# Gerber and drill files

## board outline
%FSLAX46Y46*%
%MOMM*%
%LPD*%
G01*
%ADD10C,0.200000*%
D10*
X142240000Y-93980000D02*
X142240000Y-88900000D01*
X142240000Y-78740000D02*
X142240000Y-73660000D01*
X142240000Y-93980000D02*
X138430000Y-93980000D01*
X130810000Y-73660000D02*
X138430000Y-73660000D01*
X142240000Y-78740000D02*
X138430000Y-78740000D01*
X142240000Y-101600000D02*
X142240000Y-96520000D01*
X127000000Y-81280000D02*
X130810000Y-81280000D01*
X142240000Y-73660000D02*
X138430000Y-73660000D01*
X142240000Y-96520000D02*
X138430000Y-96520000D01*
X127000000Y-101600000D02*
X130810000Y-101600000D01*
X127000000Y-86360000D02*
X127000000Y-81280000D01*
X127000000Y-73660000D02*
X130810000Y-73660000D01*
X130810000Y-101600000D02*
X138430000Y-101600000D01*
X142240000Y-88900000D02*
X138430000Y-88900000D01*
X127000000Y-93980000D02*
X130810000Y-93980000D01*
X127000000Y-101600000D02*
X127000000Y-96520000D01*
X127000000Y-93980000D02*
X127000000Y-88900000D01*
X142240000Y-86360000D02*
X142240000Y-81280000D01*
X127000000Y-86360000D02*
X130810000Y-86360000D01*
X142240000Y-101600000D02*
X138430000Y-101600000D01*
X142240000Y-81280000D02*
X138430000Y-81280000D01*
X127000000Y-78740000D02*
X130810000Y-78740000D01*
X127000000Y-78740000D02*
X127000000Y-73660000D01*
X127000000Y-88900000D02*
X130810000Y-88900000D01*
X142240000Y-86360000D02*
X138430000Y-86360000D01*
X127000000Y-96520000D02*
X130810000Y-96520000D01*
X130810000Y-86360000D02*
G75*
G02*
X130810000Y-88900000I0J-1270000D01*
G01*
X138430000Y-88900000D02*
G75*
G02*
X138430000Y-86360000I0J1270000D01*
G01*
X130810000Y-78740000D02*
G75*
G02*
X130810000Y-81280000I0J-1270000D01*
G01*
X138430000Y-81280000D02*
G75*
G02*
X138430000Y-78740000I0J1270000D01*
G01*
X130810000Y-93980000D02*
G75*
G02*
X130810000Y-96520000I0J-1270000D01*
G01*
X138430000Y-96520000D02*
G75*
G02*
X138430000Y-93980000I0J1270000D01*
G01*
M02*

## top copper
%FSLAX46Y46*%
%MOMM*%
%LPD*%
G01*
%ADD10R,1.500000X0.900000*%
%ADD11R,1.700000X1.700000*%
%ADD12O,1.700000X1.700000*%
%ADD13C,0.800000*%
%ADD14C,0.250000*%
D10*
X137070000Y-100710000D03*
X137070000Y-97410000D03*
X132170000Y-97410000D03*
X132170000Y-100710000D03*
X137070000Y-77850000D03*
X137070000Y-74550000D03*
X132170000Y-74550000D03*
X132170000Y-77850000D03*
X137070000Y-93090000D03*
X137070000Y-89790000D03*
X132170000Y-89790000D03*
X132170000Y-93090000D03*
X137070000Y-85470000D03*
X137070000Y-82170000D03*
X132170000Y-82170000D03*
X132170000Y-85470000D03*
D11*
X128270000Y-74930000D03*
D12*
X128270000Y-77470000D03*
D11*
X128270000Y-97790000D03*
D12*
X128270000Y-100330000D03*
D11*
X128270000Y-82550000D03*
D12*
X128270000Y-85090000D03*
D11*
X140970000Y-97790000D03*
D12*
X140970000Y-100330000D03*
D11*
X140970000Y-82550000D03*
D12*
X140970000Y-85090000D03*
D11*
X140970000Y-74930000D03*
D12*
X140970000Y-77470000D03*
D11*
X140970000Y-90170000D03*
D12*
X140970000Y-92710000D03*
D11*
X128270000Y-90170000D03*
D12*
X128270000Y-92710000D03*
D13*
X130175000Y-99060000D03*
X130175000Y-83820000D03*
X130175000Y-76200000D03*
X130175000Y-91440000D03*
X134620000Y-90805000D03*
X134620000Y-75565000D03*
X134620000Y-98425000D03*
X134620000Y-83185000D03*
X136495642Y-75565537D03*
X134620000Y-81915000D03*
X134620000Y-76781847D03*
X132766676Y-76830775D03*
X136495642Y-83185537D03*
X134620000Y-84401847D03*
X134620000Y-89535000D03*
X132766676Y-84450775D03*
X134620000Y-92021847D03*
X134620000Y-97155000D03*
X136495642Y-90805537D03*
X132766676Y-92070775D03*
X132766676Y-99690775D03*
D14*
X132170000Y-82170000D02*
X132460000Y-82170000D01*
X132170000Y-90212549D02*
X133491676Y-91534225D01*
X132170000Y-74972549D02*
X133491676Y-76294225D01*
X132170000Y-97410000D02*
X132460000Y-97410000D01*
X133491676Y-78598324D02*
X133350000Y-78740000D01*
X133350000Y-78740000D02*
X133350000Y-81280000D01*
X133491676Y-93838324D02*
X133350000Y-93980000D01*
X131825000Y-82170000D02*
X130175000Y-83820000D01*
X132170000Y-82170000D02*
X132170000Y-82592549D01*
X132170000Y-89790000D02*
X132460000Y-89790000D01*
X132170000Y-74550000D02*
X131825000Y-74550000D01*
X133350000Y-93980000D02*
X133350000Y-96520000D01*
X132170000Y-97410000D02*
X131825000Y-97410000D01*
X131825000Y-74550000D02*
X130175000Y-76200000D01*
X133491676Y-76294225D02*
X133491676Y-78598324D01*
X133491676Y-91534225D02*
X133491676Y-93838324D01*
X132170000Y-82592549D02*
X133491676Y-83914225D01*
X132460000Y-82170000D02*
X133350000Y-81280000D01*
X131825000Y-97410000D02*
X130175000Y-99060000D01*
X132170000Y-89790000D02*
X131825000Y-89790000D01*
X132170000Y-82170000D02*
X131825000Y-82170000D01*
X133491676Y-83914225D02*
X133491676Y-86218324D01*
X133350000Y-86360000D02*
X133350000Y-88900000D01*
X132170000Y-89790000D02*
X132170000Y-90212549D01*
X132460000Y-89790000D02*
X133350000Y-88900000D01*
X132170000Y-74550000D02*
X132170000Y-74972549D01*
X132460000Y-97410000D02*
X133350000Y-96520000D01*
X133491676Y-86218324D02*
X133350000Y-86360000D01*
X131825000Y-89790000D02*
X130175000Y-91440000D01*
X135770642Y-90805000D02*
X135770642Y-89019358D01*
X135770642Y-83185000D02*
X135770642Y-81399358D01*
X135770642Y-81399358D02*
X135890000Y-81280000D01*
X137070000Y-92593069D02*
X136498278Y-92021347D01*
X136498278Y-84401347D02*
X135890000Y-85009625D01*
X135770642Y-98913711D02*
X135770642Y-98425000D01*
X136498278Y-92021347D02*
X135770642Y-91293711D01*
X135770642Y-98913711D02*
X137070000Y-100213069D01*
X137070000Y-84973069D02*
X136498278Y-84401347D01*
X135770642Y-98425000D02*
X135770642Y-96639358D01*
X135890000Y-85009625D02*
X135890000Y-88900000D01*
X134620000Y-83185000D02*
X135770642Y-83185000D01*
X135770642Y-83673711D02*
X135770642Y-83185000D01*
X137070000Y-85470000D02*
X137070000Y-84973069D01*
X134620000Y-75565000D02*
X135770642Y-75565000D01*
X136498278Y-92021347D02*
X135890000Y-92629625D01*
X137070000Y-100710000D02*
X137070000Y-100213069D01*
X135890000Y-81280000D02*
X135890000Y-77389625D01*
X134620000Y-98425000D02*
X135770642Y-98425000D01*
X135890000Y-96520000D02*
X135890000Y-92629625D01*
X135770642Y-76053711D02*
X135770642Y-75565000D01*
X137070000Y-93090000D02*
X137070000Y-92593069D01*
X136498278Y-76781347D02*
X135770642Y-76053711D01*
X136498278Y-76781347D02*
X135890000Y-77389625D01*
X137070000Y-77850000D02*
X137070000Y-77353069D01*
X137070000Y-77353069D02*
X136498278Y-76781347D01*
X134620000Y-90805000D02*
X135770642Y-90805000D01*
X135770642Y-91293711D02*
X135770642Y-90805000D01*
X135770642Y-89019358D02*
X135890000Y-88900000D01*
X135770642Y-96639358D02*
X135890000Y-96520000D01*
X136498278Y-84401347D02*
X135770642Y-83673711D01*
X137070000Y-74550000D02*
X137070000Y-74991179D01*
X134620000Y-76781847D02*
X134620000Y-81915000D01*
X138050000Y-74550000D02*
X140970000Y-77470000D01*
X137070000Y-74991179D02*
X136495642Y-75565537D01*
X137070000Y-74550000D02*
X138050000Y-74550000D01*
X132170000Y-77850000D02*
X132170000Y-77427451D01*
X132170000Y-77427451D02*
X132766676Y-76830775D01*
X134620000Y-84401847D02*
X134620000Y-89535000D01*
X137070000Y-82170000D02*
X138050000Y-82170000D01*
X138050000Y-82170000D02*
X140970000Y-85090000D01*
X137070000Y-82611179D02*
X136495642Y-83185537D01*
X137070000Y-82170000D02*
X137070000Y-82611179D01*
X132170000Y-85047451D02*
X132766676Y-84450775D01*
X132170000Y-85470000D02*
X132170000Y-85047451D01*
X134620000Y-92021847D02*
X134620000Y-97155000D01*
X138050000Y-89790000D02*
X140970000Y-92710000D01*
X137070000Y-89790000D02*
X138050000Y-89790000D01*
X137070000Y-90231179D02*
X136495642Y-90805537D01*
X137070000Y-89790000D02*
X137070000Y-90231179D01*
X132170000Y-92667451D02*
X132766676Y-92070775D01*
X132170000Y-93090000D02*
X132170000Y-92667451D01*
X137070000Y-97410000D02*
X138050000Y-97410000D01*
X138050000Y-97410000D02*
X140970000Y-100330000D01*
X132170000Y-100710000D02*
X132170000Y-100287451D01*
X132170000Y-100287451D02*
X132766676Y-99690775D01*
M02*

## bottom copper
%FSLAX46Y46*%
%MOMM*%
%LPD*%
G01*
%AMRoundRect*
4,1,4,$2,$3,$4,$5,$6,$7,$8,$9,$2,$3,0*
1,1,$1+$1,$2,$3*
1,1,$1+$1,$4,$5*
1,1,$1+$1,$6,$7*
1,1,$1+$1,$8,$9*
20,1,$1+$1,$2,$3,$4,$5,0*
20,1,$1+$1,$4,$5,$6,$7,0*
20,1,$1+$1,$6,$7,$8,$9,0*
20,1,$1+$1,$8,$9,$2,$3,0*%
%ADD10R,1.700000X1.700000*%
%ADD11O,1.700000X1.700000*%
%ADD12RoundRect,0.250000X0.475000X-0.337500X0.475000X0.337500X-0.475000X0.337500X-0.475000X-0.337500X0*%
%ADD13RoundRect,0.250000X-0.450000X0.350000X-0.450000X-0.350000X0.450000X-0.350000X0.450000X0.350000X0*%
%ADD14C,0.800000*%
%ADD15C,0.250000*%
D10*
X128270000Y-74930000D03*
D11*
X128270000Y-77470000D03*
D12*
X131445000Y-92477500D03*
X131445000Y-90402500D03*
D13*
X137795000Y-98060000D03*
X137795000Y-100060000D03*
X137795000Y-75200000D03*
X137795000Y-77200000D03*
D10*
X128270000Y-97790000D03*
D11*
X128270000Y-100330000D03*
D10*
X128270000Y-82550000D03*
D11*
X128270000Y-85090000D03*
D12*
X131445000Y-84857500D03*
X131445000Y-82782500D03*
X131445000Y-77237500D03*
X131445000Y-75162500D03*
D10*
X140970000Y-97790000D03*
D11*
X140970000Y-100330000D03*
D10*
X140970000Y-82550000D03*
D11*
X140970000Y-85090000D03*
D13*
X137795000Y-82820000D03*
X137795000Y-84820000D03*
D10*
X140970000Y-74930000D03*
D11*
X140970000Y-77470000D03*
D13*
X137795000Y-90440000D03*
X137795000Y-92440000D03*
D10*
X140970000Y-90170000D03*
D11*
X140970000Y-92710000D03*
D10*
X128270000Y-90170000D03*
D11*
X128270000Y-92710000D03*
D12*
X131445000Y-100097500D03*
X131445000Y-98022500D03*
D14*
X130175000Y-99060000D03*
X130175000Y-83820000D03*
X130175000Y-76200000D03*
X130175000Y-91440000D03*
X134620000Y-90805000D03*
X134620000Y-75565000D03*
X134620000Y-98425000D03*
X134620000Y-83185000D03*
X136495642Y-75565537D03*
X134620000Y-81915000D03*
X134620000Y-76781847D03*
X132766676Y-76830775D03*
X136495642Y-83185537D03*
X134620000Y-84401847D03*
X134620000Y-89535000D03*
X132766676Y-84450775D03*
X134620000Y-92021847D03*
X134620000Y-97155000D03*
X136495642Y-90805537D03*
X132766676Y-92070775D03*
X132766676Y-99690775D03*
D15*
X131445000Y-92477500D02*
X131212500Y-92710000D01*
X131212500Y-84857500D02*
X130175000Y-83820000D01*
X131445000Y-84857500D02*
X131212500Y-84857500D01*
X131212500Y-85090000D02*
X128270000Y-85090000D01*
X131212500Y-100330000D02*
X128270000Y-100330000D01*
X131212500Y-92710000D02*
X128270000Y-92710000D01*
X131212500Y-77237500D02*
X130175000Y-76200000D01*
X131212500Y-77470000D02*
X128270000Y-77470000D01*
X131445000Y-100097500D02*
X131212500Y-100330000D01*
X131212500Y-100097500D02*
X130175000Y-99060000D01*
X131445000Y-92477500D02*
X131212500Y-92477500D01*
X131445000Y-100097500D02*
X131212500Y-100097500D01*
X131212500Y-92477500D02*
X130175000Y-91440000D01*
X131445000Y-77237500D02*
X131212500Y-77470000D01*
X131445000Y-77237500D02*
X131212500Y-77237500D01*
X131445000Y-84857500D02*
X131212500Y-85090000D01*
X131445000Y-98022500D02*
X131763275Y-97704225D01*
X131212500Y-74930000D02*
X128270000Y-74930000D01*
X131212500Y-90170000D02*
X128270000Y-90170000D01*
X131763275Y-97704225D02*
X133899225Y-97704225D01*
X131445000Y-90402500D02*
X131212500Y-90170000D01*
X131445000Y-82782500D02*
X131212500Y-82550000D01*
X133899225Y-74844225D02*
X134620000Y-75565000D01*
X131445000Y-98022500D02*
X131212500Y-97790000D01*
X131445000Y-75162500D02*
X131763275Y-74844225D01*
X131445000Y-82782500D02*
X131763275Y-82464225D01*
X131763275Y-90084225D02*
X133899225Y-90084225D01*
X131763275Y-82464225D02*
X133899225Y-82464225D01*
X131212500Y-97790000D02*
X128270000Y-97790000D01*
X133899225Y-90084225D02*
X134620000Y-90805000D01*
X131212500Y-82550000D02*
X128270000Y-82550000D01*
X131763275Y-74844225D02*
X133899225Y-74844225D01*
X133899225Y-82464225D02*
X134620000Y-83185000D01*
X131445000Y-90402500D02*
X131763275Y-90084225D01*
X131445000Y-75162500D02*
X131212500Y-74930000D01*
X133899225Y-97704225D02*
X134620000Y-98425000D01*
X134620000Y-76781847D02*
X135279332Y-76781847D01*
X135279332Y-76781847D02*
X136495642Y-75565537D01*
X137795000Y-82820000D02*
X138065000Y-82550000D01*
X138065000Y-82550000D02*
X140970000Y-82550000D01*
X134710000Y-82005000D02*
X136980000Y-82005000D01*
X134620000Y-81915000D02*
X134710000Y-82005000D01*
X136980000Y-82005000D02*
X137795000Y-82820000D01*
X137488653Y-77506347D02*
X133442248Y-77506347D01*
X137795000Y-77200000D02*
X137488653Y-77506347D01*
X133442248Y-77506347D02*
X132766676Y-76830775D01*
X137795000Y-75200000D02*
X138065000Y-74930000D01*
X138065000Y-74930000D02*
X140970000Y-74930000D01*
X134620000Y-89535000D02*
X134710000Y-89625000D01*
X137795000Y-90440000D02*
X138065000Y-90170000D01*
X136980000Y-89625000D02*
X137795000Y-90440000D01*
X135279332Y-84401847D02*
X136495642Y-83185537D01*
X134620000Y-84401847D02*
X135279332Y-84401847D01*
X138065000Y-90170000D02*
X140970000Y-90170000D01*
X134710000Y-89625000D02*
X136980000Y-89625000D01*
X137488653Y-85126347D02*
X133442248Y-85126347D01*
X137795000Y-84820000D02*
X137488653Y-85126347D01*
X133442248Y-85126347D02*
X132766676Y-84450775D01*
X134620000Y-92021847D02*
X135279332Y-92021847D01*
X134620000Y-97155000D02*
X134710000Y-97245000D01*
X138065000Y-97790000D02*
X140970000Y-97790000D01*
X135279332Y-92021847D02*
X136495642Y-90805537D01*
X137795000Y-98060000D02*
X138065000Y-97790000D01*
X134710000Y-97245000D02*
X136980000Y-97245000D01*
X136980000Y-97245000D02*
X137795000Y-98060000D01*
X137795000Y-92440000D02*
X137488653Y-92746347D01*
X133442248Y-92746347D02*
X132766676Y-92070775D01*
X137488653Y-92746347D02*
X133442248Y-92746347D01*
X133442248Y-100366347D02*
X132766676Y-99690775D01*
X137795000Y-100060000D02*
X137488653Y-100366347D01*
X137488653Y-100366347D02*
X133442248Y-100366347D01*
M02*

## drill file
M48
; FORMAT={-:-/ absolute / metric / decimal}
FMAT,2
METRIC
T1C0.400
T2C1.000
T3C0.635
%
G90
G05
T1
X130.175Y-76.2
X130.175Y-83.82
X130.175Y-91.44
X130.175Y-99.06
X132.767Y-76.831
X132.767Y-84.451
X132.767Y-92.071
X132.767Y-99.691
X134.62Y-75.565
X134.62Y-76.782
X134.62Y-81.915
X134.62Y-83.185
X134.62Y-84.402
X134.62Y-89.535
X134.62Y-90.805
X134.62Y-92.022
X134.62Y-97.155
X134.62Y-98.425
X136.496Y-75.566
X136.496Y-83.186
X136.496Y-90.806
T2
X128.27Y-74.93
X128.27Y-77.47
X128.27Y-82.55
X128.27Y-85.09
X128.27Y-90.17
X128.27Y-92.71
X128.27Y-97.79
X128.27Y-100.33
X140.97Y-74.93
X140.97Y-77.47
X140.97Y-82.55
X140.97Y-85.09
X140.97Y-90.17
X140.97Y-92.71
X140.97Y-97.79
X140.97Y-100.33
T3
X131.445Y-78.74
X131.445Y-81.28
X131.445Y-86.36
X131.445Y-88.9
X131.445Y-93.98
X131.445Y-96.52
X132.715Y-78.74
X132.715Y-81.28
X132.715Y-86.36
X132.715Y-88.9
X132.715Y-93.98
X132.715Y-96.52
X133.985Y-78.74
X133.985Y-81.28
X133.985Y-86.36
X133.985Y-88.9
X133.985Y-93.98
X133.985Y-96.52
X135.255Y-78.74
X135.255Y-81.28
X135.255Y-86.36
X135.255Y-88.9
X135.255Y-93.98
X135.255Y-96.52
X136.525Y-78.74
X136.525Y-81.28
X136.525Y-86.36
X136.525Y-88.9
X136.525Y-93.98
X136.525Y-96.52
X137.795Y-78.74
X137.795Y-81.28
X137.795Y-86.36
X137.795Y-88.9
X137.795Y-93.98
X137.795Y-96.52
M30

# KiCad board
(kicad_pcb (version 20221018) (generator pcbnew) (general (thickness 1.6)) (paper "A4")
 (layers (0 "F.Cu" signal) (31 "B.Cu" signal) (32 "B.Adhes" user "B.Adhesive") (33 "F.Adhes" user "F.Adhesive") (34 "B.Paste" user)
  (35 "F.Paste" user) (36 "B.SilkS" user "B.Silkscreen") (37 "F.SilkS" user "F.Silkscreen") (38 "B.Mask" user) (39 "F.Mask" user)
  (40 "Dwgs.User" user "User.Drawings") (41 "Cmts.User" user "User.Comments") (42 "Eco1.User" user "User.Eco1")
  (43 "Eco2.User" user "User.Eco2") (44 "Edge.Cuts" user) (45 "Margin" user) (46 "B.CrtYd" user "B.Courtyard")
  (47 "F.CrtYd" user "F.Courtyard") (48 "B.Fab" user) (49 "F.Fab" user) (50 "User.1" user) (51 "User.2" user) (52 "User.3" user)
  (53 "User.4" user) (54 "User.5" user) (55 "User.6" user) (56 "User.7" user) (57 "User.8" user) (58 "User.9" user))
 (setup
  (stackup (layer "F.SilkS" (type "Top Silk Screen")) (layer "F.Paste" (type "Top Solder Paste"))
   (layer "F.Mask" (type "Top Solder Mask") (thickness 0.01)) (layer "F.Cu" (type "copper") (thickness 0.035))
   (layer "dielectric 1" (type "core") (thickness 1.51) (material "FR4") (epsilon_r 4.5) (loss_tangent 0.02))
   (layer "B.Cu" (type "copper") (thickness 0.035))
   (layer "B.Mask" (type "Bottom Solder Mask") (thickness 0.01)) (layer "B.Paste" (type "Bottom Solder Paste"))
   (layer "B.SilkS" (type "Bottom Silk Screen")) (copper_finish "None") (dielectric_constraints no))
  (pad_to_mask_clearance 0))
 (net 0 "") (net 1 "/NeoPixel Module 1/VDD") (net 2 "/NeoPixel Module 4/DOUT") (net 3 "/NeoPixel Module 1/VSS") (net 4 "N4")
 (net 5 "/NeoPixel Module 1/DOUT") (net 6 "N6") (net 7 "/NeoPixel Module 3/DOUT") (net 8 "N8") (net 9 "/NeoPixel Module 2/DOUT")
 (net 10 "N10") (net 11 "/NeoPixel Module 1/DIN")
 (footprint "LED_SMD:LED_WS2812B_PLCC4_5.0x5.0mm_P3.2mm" (layer "F.Cu") (at 134.62 99.06 180)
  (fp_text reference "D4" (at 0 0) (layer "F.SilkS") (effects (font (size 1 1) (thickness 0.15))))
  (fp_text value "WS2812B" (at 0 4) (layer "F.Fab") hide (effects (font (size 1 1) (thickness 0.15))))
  (pad "1" smd rect (at -2.45 -1.65 180) (size 1.5 0.9) (layers "F.Cu" "F.Paste" "F.Mask") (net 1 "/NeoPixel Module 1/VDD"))
  (pad "2" smd rect (at -2.45 1.65 180) (size 1.5 0.9) (layers "F.Cu" "F.Paste" "F.Mask") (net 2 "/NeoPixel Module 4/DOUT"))
  (pad "3" smd rect (at 2.45 1.65 180) (size 1.5 0.9) (layers "F.Cu" "F.Paste" "F.Mask") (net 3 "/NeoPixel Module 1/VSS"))
  (pad "4" smd rect (at 2.45 -1.65 180) (size 1.5 0.9) (layers "F.Cu" "F.Paste" "F.Mask") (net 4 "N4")))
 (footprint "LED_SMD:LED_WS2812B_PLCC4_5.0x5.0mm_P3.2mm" (layer "F.Cu") (at 134.62 76.2 180)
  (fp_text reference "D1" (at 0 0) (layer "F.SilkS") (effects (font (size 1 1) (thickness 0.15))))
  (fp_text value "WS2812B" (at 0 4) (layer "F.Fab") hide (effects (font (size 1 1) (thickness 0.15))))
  (pad "1" smd rect (at -2.45 -1.65 180) (size 1.5 0.9) (layers "F.Cu" "F.Paste" "F.Mask") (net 1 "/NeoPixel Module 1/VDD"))
  (pad "2" smd rect (at -2.45 1.65 180) (size 1.5 0.9) (layers "F.Cu" "F.Paste" "F.Mask") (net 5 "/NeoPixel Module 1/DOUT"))
  (pad "3" smd rect (at 2.45 1.65 180) (size 1.5 0.9) (layers "F.Cu" "F.Paste" "F.Mask") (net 3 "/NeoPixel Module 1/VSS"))
  (pad "4" smd rect (at 2.45 -1.65 180) (size 1.5 0.9) (layers "F.Cu" "F.Paste" "F.Mask") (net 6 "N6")))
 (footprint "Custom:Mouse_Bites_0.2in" (layer "F.Cu") (at 134.62 87.63)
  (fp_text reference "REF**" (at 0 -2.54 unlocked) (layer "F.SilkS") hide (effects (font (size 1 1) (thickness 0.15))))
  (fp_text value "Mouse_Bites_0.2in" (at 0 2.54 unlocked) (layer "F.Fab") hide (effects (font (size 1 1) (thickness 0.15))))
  (fp_arc (start -3.81 -1.27) (mid -2.54 0) (end -3.81 1.27) (stroke (width 0.2) (type default)) (layer "Edge.Cuts"))
  (fp_arc (start 3.81 1.27) (mid 2.54 0) (end 3.81 -1.27) (stroke (width 0.2) (type default)) (layer "Edge.Cuts"))
  (pad "" np_thru_hole circle (at -3.175 -1.27) (size 0.635 0.635) (drill 0.635) (layers "*.Mask") (thermal_bridge_angle 90))
  (pad "" np_thru_hole circle (at -3.175 1.27) (size 0.635 0.635) (drill 0.635) (layers "*.Mask") (thermal_bridge_angle 90))
  (pad "" np_thru_hole circle (at -1.905 -1.27) (size 0.635 0.635) (drill 0.635) (layers "*.Mask") (thermal_bridge_angle 90))
  (pad "" np_thru_hole circle (at -1.905 1.27) (size 0.635 0.635) (drill 0.635) (layers "*.Mask") (thermal_bridge_angle 90))
  (pad "" np_thru_hole circle (at -0.635 -1.27) (size 0.635 0.635) (drill 0.635) (layers "*.Mask") (thermal_bridge_angle 90))
  (pad "" np_thru_hole circle (at -0.635 1.27) (size 0.635 0.635) (drill 0.635) (layers "*.Mask") (thermal_bridge_angle 90))
  (pad "" np_thru_hole circle (at 0.635 -1.27) (size 0.635 0.635) (drill 0.635) (layers "*.Mask") (thermal_bridge_angle 90))
  (pad "" np_thru_hole circle (at 0.635 1.27) (size 0.635 0.635) (drill 0.635) (layers "*.Mask") (thermal_bridge_angle 90))
  (pad "" np_thru_hole circle (at 1.905 -1.27) (size 0.635 0.635) (drill 0.635) (layers "*.Mask") (thermal_bridge_angle 90))
  (pad "" np_thru_hole circle (at 1.905 1.27) (size 0.635 0.635) (drill 0.635) (layers "*.Mask") (thermal_bridge_angle 90))
  (pad "" np_thru_hole circle (at 3.175 -1.27) (size 0.635 0.635) (drill 0.635) (layers "*.Mask") (thermal_bridge_angle 90))
  (pad "" np_thru_hole circle (at 3.175 1.27) (size 0.635 0.635) (drill 0.635) (layers "*.Mask") (thermal_bridge_angle 90)))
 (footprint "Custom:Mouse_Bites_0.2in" (layer "F.Cu") (at 134.62 80.01)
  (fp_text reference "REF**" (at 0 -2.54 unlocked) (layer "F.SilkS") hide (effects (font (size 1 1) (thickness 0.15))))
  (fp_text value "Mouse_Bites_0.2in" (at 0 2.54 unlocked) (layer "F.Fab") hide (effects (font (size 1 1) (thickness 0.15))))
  (fp_arc (start -3.81 -1.27) (mid -2.54 0) (end -3.81 1.27) (stroke (width 0.2) (type default)) (layer "Edge.Cuts"))
  (fp_arc (start 3.81 1.27) (mid 2.54 0) (end 3.81 -1.27) (stroke (width 0.2) (type default)) (layer "Edge.Cuts"))
  (pad "" np_thru_hole circle (at -3.175 -1.27) (size 0.635 0.635) (drill 0.635) (layers "*.Mask") (thermal_bridge_angle 90))
  (pad "" np_thru_hole circle (at -3.175 1.27) (size 0.635 0.635) (drill 0.635) (layers "*.Mask") (thermal_bridge_angle 90))
  (pad "" np_thru_hole circle (at -1.905 -1.27) (size 0.635 0.635) (drill 0.635) (layers "*.Mask") (thermal_bridge_angle 90))
  (pad "" np_thru_hole circle (at -1.905 1.27) (size 0.635 0.635) (drill 0.635) (layers "*.Mask") (thermal_bridge_angle 90))
  (pad "" np_thru_hole circle (at -0.635 -1.27) (size 0.635 0.635) (drill 0.635) (layers "*.Mask") (thermal_bridge_angle 90))
  (pad "" np_thru_hole circle (at -0.635 1.27) (size 0.635 0.635) (drill 0.635) (layers "*.Mask") (thermal_bridge_angle 90))
  (pad "" np_thru_hole circle (at 0.635 -1.27) (size 0.635 0.635) (drill 0.635) (layers "*.Mask") (thermal_bridge_angle 90))
  (pad "" np_thru_hole circle (at 0.635 1.27) (size 0.635 0.635) (drill 0.635) (layers "*.Mask") (thermal_bridge_angle 90))
  (pad "" np_thru_hole circle (at 1.905 -1.27) (size 0.635 0.635) (drill 0.635) (layers "*.Mask") (thermal_bridge_angle 90))
  (pad "" np_thru_hole circle (at 1.905 1.27) (size 0.635 0.635) (drill 0.635) (layers "*.Mask") (thermal_bridge_angle 90))
  (pad "" np_thru_hole circle (at 3.175 -1.27) (size 0.635 0.635) (drill 0.635) (layers "*.Mask") (thermal_bridge_angle 90))
  (pad "" np_thru_hole circle (at 3.175 1.27) (size 0.635 0.635) (drill 0.635) (layers "*.Mask") (thermal_bridge_angle 90)))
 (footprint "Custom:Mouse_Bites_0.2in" (layer "F.Cu") (at 134.62 95.25)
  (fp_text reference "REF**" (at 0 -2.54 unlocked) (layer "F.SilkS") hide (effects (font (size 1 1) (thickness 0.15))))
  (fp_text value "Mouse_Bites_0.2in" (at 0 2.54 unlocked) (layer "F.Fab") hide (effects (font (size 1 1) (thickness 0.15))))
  (fp_arc (start -3.81 -1.27) (mid -2.54 0) (end -3.81 1.27) (stroke (width 0.2) (type default)) (layer "Edge.Cuts"))
  (fp_arc (start 3.81 1.27) (mid 2.54 0) (end 3.81 -1.27) (stroke (width 0.2) (type default)) (layer "Edge.Cuts"))
  (pad "" np_thru_hole circle (at -3.175 -1.27) (size 0.635 0.635) (drill 0.635) (layers "*.Mask") (thermal_bridge_angle 90))
  (pad "" np_thru_hole circle (at -3.175 1.27) (size 0.635 0.635) (drill 0.635) (layers "*.Mask") (thermal_bridge_angle 90))
  (pad "" np_thru_hole circle (at -1.905 -1.27) (size 0.635 0.635) (drill 0.635) (layers "*.Mask") (thermal_bridge_angle 90))
  (pad "" np_thru_hole circle (at -1.905 1.27) (size 0.635 0.635) (drill 0.635) (layers "*.Mask") (thermal_bridge_angle 90))
  (pad "" np_thru_hole circle (at -0.635 -1.27) (size 0.635 0.635) (drill 0.635) (layers "*.Mask") (thermal_bridge_angle 90))
  (pad "" np_thru_hole circle (at -0.635 1.27) (size 0.635 0.635) (drill 0.635) (layers "*.Mask") (thermal_bridge_angle 90))
  (pad "" np_thru_hole circle (at 0.635 -1.27) (size 0.635 0.635) (drill 0.635) (layers "*.Mask") (thermal_bridge_angle 90))
  (pad "" np_thru_hole circle (at 0.635 1.27) (size 0.635 0.635) (drill 0.635) (layers "*.Mask") (thermal_bridge_angle 90))
  (pad "" np_thru_hole circle (at 1.905 -1.27) (size 0.635 0.635) (drill 0.635) (layers "*.Mask") (thermal_bridge_angle 90))
  (pad "" np_thru_hole circle (at 1.905 1.27) (size 0.635 0.635) (drill 0.635) (layers "*.Mask") (thermal_bridge_angle 90))
  (pad "" np_thru_hole circle (at 3.175 -1.27) (size 0.635 0.635) (drill 0.635) (layers "*.Mask") (thermal_bridge_angle 90))
  (pad "" np_thru_hole circle (at 3.175 1.27) (size 0.635 0.635) (drill 0.635) (layers "*.Mask") (thermal_bridge_angle 90)))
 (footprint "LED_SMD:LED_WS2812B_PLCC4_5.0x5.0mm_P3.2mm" (layer "F.Cu") (at 134.62 91.44 180)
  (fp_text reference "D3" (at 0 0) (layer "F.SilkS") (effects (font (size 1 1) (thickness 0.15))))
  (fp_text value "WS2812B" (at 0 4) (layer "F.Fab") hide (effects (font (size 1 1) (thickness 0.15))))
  (pad "1" smd rect (at -2.45 -1.65 180) (size 1.5 0.9) (layers "F.Cu" "F.Paste" "F.Mask") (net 1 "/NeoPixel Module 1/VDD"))
  (pad "2" smd rect (at -2.45 1.65 180) (size 1.5 0.9) (layers "F.Cu" "F.Paste" "F.Mask") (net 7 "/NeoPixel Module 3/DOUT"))
  (pad "3" smd rect (at 2.45 1.65 180) (size 1.5 0.9) (layers "F.Cu" "F.Paste" "F.Mask") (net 3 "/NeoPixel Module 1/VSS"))
  (pad "4" smd rect (at 2.45 -1.65 180) (size 1.5 0.9) (layers "F.Cu" "F.Paste" "F.Mask") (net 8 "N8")))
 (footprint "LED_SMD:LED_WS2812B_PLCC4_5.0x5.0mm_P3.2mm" (layer "F.Cu") (at 134.62 83.82 180)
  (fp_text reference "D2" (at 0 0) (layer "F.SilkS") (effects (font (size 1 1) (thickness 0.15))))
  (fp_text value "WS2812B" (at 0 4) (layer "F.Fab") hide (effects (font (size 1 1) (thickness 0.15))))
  (pad "1" smd rect (at -2.45 -1.65 180) (size 1.5 0.9) (layers "F.Cu" "F.Paste" "F.Mask") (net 1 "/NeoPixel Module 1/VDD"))
  (pad "2" smd rect (at -2.45 1.65 180) (size 1.5 0.9) (layers "F.Cu" "F.Paste" "F.Mask") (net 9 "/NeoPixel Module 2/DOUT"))
  (pad "3" smd rect (at 2.45 1.65 180) (size 1.5 0.9) (layers "F.Cu" "F.Paste" "F.Mask") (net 3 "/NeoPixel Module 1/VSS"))
  (pad "4" smd rect (at 2.45 -1.65 180) (size 1.5 0.9) (layers "F.Cu" "F.Paste" "F.Mask") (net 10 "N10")))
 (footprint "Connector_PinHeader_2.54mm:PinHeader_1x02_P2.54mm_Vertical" (layer "B.Cu") (at 128.27 74.93 180)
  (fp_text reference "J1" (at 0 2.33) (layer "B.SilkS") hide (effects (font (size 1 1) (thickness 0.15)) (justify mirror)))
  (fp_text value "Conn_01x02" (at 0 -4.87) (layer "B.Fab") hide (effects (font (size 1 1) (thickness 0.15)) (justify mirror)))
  (pad "1" thru_hole rect (at 0 0 180) (size 1.7 1.7) (drill 1) (layers "*.Cu" "*.Mask") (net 1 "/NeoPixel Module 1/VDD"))
  (pad "2" thru_hole oval (at 0 -2.54 180) (size 1.7 1.7) (drill 1) (layers "*.Cu" "*.Mask") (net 3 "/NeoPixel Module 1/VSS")))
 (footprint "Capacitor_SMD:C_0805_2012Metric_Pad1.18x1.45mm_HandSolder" (layer "B.Cu") (at 131.445 91.44 90)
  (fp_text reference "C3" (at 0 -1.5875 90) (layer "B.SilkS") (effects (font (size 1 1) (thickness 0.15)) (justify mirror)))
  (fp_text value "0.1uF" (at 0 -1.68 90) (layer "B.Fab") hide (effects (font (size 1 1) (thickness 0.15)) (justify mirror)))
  (pad "1" smd roundrect (at -1.0375 0 90) (size 1.175 1.45) (layers "B.Cu" "B.Paste" "B.Mask") (roundrect_rratio 0.212766)
   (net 3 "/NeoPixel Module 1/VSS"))
  (pad "2" smd roundrect (at 1.0375 0 90) (size 1.175 1.45) (layers "B.Cu" "B.Paste" "B.Mask") (roundrect_rratio 0.212766)
   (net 1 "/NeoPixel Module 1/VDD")))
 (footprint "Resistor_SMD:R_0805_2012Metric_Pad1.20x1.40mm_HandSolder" (layer "B.Cu") (at 137.795 99.06 -90)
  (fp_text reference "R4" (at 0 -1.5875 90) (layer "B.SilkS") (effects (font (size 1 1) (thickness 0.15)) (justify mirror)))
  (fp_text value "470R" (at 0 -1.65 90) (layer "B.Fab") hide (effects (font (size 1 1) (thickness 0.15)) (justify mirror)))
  (pad "1" smd roundrect (at -1 0 270) (size 1.2 1.4) (layers "B.Cu" "B.Paste" "B.Mask") (roundrect_rratio 0.208333)
   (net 7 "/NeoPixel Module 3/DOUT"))
  (pad "2" smd roundrect (at 1 0 270) (size 1.2 1.4) (layers "B.Cu" "B.Paste" "B.Mask") (roundrect_rratio 0.208333) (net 4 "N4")))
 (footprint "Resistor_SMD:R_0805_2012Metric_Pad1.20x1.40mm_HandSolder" (layer "B.Cu") (at 137.795 76.2 -90)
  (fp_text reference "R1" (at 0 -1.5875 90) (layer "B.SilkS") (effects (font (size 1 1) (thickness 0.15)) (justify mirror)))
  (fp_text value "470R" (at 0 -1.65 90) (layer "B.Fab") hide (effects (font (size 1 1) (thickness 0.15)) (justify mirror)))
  (pad "1" smd roundrect (at -1 0 270) (size 1.2 1.4) (layers "B.Cu" "B.Paste" "B.Mask") (roundrect_rratio 0.208333)
   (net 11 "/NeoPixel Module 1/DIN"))
  (pad "2" smd roundrect (at 1 0 270) (size 1.2 1.4) (layers "B.Cu" "B.Paste" "B.Mask") (roundrect_rratio 0.208333) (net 6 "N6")))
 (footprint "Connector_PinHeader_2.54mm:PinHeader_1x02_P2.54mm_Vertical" (layer "B.Cu") (at 128.27 97.79 180)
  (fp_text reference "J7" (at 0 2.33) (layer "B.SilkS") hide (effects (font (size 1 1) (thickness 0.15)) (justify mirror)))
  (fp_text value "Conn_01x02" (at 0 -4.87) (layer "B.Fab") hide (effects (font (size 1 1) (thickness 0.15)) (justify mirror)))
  (pad "1" thru_hole rect (at 0 0 180) (size 1.7 1.7) (drill 1) (layers "*.Cu" "*.Mask") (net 1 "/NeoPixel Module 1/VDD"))
  (pad "2" thru_hole oval (at 0 -2.54 180) (size 1.7 1.7) (drill 1) (layers "*.Cu" "*.Mask") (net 3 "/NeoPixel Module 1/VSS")))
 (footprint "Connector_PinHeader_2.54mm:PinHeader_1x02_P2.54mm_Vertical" (layer "B.Cu") (at 128.27 82.55 180)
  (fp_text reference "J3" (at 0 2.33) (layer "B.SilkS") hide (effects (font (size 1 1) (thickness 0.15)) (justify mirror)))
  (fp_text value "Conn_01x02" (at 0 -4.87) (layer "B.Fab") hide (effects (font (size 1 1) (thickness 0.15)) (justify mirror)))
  (pad "1" thru_hole rect (at 0 0 180) (size 1.7 1.7) (drill 1) (layers "*.Cu" "*.Mask") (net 1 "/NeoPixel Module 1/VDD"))
  (pad "2" thru_hole oval (at 0 -2.54 180) (size 1.7 1.7) (drill 1) (layers "*.Cu" "*.Mask") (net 3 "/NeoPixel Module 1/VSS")))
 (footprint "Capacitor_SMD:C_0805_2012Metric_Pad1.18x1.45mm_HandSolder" (layer "B.Cu") (at 131.445 83.82 90)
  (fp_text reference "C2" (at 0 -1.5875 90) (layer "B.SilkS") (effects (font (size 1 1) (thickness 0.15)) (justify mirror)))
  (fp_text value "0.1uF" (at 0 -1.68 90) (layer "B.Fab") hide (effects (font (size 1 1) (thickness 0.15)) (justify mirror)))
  (pad "1" smd roundrect (at -1.0375 0 90) (size 1.175 1.45) (layers "B.Cu" "B.Paste" "B.Mask") (roundrect_rratio 0.212766)
   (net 3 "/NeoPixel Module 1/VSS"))
  (pad "2" smd roundrect (at 1.0375 0 90) (size 1.175 1.45) (layers "B.Cu" "B.Paste" "B.Mask") (roundrect_rratio 0.212766)
   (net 1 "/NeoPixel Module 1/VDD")))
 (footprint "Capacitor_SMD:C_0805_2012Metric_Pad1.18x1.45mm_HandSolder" (layer "B.Cu") (at 131.445 76.2 90)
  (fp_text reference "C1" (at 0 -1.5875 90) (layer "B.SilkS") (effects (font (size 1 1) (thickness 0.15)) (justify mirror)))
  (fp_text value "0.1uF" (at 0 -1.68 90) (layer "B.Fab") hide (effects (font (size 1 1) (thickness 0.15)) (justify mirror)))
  (pad "1" smd roundrect (at -1.0375 0 90) (size 1.175 1.45) (layers "B.Cu" "B.Paste" "B.Mask") (roundrect_rratio 0.212766)
   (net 3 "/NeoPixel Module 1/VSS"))
  (pad "2" smd roundrect (at 1.0375 0 90) (size 1.175 1.45) (layers "B.Cu" "B.Paste" "B.Mask") (roundrect_rratio 0.212766)
   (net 1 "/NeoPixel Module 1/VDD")))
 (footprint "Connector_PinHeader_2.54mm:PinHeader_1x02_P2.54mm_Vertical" (layer "B.Cu") (at 140.97 97.79 180)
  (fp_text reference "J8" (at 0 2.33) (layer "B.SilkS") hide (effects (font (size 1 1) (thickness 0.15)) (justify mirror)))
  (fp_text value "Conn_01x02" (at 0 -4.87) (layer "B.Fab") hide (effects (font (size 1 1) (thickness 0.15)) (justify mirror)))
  (pad "1" thru_hole rect (at 0 0 180) (size 1.7 1.7) (drill 1) (layers "*.Cu" "*.Mask") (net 7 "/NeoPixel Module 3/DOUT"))
  (pad "2" thru_hole oval (at 0 -2.54 180) (size 1.7 1.7) (drill 1) (layers "*.Cu" "*.Mask") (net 2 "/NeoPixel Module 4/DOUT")))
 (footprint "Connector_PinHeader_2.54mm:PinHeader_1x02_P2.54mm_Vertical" (layer "B.Cu") (at 140.97 82.55 180)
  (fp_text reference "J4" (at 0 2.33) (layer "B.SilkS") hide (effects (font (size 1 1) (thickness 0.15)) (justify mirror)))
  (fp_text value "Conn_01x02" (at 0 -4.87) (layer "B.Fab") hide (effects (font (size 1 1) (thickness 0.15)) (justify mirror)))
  (pad "1" thru_hole rect (at 0 0 180) (size 1.7 1.7) (drill 1) (layers "*.Cu" "*.Mask") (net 5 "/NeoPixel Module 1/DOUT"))
  (pad "2" thru_hole oval (at 0 -2.54 180) (size 1.7 1.7) (drill 1) (layers "*.Cu" "*.Mask") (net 9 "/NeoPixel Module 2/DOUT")))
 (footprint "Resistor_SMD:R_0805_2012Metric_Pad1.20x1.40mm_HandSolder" (layer "B.Cu") (at 137.795 83.82 -90)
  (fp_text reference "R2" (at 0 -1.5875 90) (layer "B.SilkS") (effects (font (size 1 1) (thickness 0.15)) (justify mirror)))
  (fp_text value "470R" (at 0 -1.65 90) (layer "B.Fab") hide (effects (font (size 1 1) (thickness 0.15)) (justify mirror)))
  (pad "1" smd roundrect (at -1 0 270) (size 1.2 1.4) (layers "B.Cu" "B.Paste" "B.Mask") (roundrect_rratio 0.208333)
   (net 5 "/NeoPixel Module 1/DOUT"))
  (pad "2" smd roundrect (at 1 0 270) (size 1.2 1.4) (layers "B.Cu" "B.Paste" "B.Mask") (roundrect_rratio 0.208333) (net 10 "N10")))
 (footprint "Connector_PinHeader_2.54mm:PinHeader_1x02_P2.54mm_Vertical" (layer "B.Cu") (at 140.97 74.93 180)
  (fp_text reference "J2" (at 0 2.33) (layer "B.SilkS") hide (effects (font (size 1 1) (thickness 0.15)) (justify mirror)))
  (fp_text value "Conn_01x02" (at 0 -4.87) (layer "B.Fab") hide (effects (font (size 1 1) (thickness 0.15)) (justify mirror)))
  (pad "1" thru_hole rect (at 0 0 180) (size 1.7 1.7) (drill 1) (layers "*.Cu" "*.Mask") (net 11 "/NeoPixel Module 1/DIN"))
  (pad "2" thru_hole oval (at 0 -2.54 180) (size 1.7 1.7) (drill 1) (layers "*.Cu" "*.Mask") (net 5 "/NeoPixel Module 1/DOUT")))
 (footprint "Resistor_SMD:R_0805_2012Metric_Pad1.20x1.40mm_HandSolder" (layer "B.Cu") (at 137.795 91.44 -90)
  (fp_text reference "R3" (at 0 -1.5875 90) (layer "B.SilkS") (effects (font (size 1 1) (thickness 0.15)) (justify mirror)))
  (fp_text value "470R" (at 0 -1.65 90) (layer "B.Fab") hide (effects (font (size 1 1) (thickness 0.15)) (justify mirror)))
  (pad "1" smd roundrect (at -1 0 270) (size 1.2 1.4) (layers "B.Cu" "B.Paste" "B.Mask") (roundrect_rratio 0.208333)
   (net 9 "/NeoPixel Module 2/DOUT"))
  (pad "2" smd roundrect (at 1 0 270) (size 1.2 1.4) (layers "B.Cu" "B.Paste" "B.Mask") (roundrect_rratio 0.208333) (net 8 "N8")))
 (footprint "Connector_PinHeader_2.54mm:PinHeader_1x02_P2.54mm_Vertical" (layer "B.Cu") (at 140.97 90.17 180)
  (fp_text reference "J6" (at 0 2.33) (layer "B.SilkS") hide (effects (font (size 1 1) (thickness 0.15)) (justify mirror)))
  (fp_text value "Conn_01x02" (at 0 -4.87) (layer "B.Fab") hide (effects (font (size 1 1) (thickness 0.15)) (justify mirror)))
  (pad "1" thru_hole rect (at 0 0 180) (size 1.7 1.7) (drill 1) (layers "*.Cu" "*.Mask") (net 9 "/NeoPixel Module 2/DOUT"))
  (pad "2" thru_hole oval (at 0 -2.54 180) (size 1.7 1.7) (drill 1) (layers "*.Cu" "*.Mask") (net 7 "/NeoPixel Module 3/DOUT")))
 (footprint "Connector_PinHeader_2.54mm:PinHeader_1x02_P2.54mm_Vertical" (layer "B.Cu") (at 128.27 90.17 180)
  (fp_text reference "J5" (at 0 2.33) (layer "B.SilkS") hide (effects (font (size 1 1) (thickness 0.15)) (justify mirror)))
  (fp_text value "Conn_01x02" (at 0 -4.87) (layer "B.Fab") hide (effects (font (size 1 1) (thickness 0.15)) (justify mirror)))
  (pad "1" thru_hole rect (at 0 0 180) (size 1.7 1.7) (drill 1) (layers "*.Cu" "*.Mask") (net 1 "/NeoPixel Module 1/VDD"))
  (pad "2" thru_hole oval (at 0 -2.54 180) (size 1.7 1.7) (drill 1) (layers "*.Cu" "*.Mask") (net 3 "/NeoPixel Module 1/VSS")))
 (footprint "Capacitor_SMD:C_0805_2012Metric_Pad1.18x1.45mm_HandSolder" (layer "B.Cu") (at 131.445 99.06 90)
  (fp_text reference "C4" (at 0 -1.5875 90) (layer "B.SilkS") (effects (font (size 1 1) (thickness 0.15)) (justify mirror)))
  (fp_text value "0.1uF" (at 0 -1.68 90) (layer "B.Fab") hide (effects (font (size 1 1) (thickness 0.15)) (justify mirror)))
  (pad "1" smd roundrect (at -1.0375 0 90) (size 1.175 1.45) (layers "B.Cu" "B.Paste" "B.Mask") (roundrect_rratio 0.212766)
   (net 3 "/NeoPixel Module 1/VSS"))
  (pad "2" smd roundrect (at 1.0375 0 90) (size 1.175 1.45) (layers "B.Cu" "B.Paste" "B.Mask") (roundrect_rratio 0.212766)
   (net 1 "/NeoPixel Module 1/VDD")))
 (gr_line (start 142.24 93.98) (end 142.24 88.9) (stroke (width 0.2) (type default)) (layer "Edge.Cuts"))
 (gr_line (start 142.24 78.74) (end 142.24 73.66) (stroke (width 0.2) (type default)) (layer "Edge.Cuts"))
 (gr_line (start 142.24 93.98) (end 138.43 93.98) (stroke (width 0.2) (type default)) (layer "Edge.Cuts"))
 (gr_line (start 130.81 73.66) (end 138.43 73.66) (stroke (width 0.2) (type default)) (layer "Edge.Cuts"))
 (gr_line (start 142.24 78.74) (end 138.43 78.74) (stroke (width 0.2) (type default)) (layer "Edge.Cuts"))
 (gr_line (start 142.24 101.6) (end 142.24 96.52) (stroke (width 0.2) (type default)) (layer "Edge.Cuts"))
 (gr_line (start 127 81.28) (end 130.81 81.28) (stroke (width 0.2) (type default)) (layer "Edge.Cuts"))
 (gr_line (start 142.24 73.66) (end 138.43 73.66) (stroke (width 0.2) (type default)) (layer "Edge.Cuts"))
 (gr_line (start 142.24 96.52) (end 138.43 96.52) (stroke (width 0.2) (type default)) (layer "Edge.Cuts"))
 (gr_line (start 127 101.6) (end 130.81 101.6) (stroke (width 0.2) (type default)) (layer "Edge.Cuts"))
 (gr_line (start 127 86.36) (end 127 81.28) (stroke (width 0.2) (type default)) (layer "Edge.Cuts"))
 (gr_line (start 127 73.66) (end 130.81 73.66) (stroke (width 0.2) (type default)) (layer "Edge.Cuts"))
 (gr_line (start 130.81 101.6) (end 138.43 101.6) (stroke (width 0.2) (type default)) (layer "Edge.Cuts"))
 (gr_line (start 142.24 88.9) (end 138.43 88.9) (stroke (width 0.2) (type default)) (layer "Edge.Cuts"))
 (gr_line (start 127 93.98) (end 130.81 93.98) (stroke (width 0.2) (type default)) (layer "Edge.Cuts"))
 (gr_line (start 127 101.6) (end 127 96.52) (stroke (width 0.2) (type default)) (layer "Edge.Cuts"))
 (gr_line (start 127 93.98) (end 127 88.9) (stroke (width 0.2) (type default)) (layer "Edge.Cuts"))
 (gr_line (start 142.24 86.36) (end 142.24 81.28) (stroke (width 0.2) (type default)) (layer "Edge.Cuts"))
 (gr_line (start 127 86.36) (end 130.81 86.36) (stroke (width 0.2) (type default)) (layer "Edge.Cuts"))
 (gr_line (start 142.24 101.6) (end 138.43 101.6) (stroke (width 0.2) (type default)) (layer "Edge.Cuts"))
 (gr_line (start 142.24 81.28) (end 138.43 81.28) (stroke (width 0.2) (type default)) (layer "Edge.Cuts"))
 (gr_line (start 127 78.74) (end 130.81 78.74) (stroke (width 0.2) (type default)) (layer "Edge.Cuts"))
 (gr_line (start 127 78.74) (end 127 73.66) (stroke (width 0.2) (type default)) (layer "Edge.Cuts"))
 (gr_line (start 127 88.9) (end 130.81 88.9) (stroke (width 0.2) (type default)) (layer "Edge.Cuts"))
 (gr_line (start 142.24 86.36) (end 138.43 86.36) (stroke (width 0.2) (type default)) (layer "Edge.Cuts"))
 (gr_line (start 127 96.52) (end 130.81 96.52) (stroke (width 0.2) (type default)) (layer "Edge.Cuts"))
 (segment (start 132.17 82.17) (end 132.46 82.17) (width 0.25) (layer "F.Cu") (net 3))
 (segment (start 132.17 90.212549) (end 133.491676 91.534225) (width 0.25) (layer "F.Cu") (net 3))
 (segment (start 132.17 74.972549) (end 133.491676 76.294225) (width 0.25) (layer "F.Cu") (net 3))
 (segment (start 132.17 97.41) (end 132.46 97.41) (width 0.25) (layer "F.Cu") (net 3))
 (segment (start 133.491676 78.598324) (end 133.35 78.74) (width 0.25) (layer "F.Cu") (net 3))
 (segment (start 133.35 78.74) (end 133.35 81.28) (width 0.25) (layer "F.Cu") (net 3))
 (segment (start 133.491676 93.838324) (end 133.35 93.98) (width 0.25) (layer "F.Cu") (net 3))
 (segment (start 131.825 82.17) (end 130.175 83.82) (width 0.25) (layer "F.Cu") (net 3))
 (segment (start 132.17 82.17) (end 132.17 82.592549) (width 0.25) (layer "F.Cu") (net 3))
 (segment (start 132.17 89.79) (end 132.46 89.79) (width 0.25) (layer "F.Cu") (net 3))
 (segment (start 132.17 74.55) (end 131.825 74.55) (width 0.25) (layer "F.Cu") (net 3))
 (segment (start 133.35 93.98) (end 133.35 96.52) (width 0.25) (layer "F.Cu") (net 3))
 (segment (start 132.17 97.41) (end 131.825 97.41) (width 0.25) (layer "F.Cu") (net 3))
 (segment (start 131.825 74.55) (end 130.175 76.2) (width 0.25) (layer "F.Cu") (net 3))
 (segment (start 133.491676 76.294225) (end 133.491676 78.598324) (width 0.25) (layer "F.Cu") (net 3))
 (segment (start 133.491676 91.534225) (end 133.491676 93.838324) (width 0.25) (layer "F.Cu") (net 3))
 (segment (start 132.17 82.592549) (end 133.491676 83.914225) (width 0.25) (layer "F.Cu") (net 3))
 (segment (start 132.46 82.17) (end 133.35 81.28) (width 0.25) (layer "F.Cu") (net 3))
 (segment (start 131.825 97.41) (end 130.175 99.06) (width 0.25) (layer "F.Cu") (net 3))
 (segment (start 132.17 89.79) (end 131.825 89.79) (width 0.25) (layer "F.Cu") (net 3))
 (segment (start 132.17 82.17) (end 131.825 82.17) (width 0.25) (layer "F.Cu") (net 3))
 (segment (start 133.491676 83.914225) (end 133.491676 86.218324) (width 0.25) (layer "F.Cu") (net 3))
 (segment (start 133.35 86.36) (end 133.35 88.9) (width 0.25) (layer "F.Cu") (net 3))
 (segment (start 132.17 89.79) (end 132.17 90.212549) (width 0.25) (layer "F.Cu") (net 3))
 (segment (start 132.46 89.79) (end 133.35 88.9) (width 0.25) (layer "F.Cu") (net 3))
 (segment (start 132.17 74.55) (end 132.17 74.972549) (width 0.25) (layer "F.Cu") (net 3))
 (segment (start 132.46 97.41) (end 133.35 96.52) (width 0.25) (layer "F.Cu") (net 3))
 (segment (start 133.491676 86.218324) (end 133.35 86.36) (width 0.25) (layer "F.Cu") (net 3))
 (segment (start 131.825 89.79) (end 130.175 91.44) (width 0.25) (layer "F.Cu") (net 3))
 (via (at 130.175 99.06) (size 0.8) (drill 0.4) (layers "F.Cu" "B.Cu") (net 3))
 (via (at 130.175 83.82) (size 0.8) (drill 0.4) (layers "F.Cu" "B.Cu") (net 3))
 (via (at 130.175 76.2) (size 0.8) (drill 0.4) (layers "F.Cu" "B.Cu") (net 3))
 (via (at 130.175 91.44) (size 0.8) (drill 0.4) (layers "F.Cu" "B.Cu") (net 3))
 (segment (start 131.445 92.4775) (end 131.2125 92.71) (width 0.25) (layer "B.Cu") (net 3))
 (segment (start 131.2125 84.8575) (end 130.175 83.82) (width 0.25) (layer "B.Cu") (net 3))
 (segment (start 131.445 84.8575) (end 131.2125 84.8575) (width 0.25) (layer "B.Cu") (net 3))
 (segment (start 131.2125 85.09) (end 128.27 85.09) (width 0.25) (layer "B.Cu") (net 3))
 (segment (start 131.2125 100.33) (end 128.27 100.33) (width 0.25) (layer "B.Cu") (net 3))
 (segment (start 131.2125 92.71) (end 128.27 92.71) (width 0.25) (layer "B.Cu") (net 3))
 (segment (start 131.2125 77.2375) (end 130.175 76.2) (width 0.25) (layer "B.Cu") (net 3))
 (segment (start 131.2125 77.47) (end 128.27 77.47) (width 0.25) (layer "B.Cu") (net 3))
 (segment (start 131.445 100.0975) (end 131.2125 100.33) (width 0.25) (layer "B.Cu") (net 3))
 (segment (start 131.2125 100.0975) (end 130.175 99.06) (width 0.25) (layer "B.Cu") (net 3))
 (segment (start 131.445 92.4775) (end 131.2125 92.4775) (width 0.25) (layer "B.Cu") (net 3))
 (segment (start 131.445 100.0975) (end 131.2125 100.0975) (width 0.25) (layer "B.Cu") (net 3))
 (segment (start 131.2125 92.4775) (end 130.175 91.44) (width 0.25) (layer "B.Cu") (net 3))
 (segment (start 131.445 77.2375) (end 131.2125 77.47) (width 0.25) (layer "B.Cu") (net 3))
 (segment (start 131.445 77.2375) (end 131.2125 77.2375) (width 0.25) (layer "B.Cu") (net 3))
 (segment (start 131.445 84.8575) (end 131.2125 85.09) (width 0.25) (layer "B.Cu") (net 3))
 (segment (start 135.770642 90.805) (end 135.770642 89.019358) (width 0.25) (layer "F.Cu") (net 1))
 (segment (start 135.770642 83.185) (end 135.770642 81.399358) (width 0.25) (layer "F.Cu") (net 1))
 (segment (start 135.770642 81.399358) (end 135.89 81.28) (width 0.25) (layer "F.Cu") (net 1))
 (segment (start 137.07 92.593069) (end 136.498278 92.021347) (width 0.25) (layer "F.Cu") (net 1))
 (segment (start 136.498278 84.401347) (end 135.89 85.009625) (width 0.25) (layer "F.Cu") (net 1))
 (segment (start 135.770642 98.913711) (end 135.770642 98.425) (width 0.25) (layer "F.Cu") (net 1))
 (segment (start 136.498278 92.021347) (end 135.770642 91.293711) (width 0.25) (layer "F.Cu") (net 1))
 (segment (start 135.770642 98.913711) (end 137.07 100.213069) (width 0.25) (layer "F.Cu") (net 1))
 (segment (start 137.07 84.973069) (end 136.498278 84.401347) (width 0.25) (layer "F.Cu") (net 1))
 (segment (start 135.770642 98.425) (end 135.770642 96.639358) (width 0.25) (layer "F.Cu") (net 1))
 (segment (start 135.89 85.009625) (end 135.89 88.9) (width 0.25) (layer "F.Cu") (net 1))
 (segment (start 134.62 83.185) (end 135.770642 83.185) (width 0.25) (layer "F.Cu") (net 1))
 (segment (start 135.770642 83.673711) (end 135.770642 83.185) (width 0.25) (layer "F.Cu") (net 1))
 (segment (start 137.07 85.47) (end 137.07 84.973069) (width 0.25) (layer "F.Cu") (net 1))
 (segment (start 134.62 75.565) (end 135.770642 75.565) (width 0.25) (layer "F.Cu") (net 1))
 (segment (start 136.498278 92.021347) (end 135.89 92.629625) (width 0.25) (layer "F.Cu") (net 1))
 (segment (start 137.07 100.71) (end 137.07 100.213069) (width 0.25) (layer "F.Cu") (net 1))
 (segment (start 135.89 81.28) (end 135.89 77.389625) (width 0.25) (layer "F.Cu") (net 1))
 (segment (start 134.62 98.425) (end 135.770642 98.425) (width 0.25) (layer "F.Cu") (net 1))
 (segment (start 135.89 96.52) (end 135.89 92.629625) (width 0.25) (layer "F.Cu") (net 1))
 (segment (start 135.770642 76.053711) (end 135.770642 75.565) (width 0.25) (layer "F.Cu") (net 1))
 (segment (start 137.07 93.09) (end 137.07 92.593069) (width 0.25) (layer "F.Cu") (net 1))
 (segment (start 136.498278 76.781347) (end 135.770642 76.053711) (width 0.25) (layer "F.Cu") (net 1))
 (segment (start 136.498278 76.781347) (end 135.89 77.389625) (width 0.25) (layer "F.Cu") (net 1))
 (segment (start 137.07 77.85) (end 137.07 77.353069) (width 0.25) (layer "F.Cu") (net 1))
 (segment (start 137.07 77.353069) (end 136.498278 76.781347) (width 0.25) (layer "F.Cu") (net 1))
 (segment (start 134.62 90.805) (end 135.770642 90.805) (width 0.25) (layer "F.Cu") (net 1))
 (segment (start 135.770642 91.293711) (end 135.770642 90.805) (width 0.25) (layer "F.Cu") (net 1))
 (segment (start 135.770642 89.019358) (end 135.89 88.9) (width 0.25) (layer "F.Cu") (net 1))
 (segment (start 135.770642 96.639358) (end 135.89 96.52) (width 0.25) (layer "F.Cu") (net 1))
 (segment (start 136.498278 84.401347) (end 135.770642 83.673711) (width 0.25) (layer "F.Cu") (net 1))
 (via (at 134.62 90.805) (size 0.8) (drill 0.4) (layers "F.Cu" "B.Cu") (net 1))
 (via (at 134.62 75.565) (size 0.8) (drill 0.4) (layers "F.Cu" "B.Cu") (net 1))
 (via (at 134.62 98.425) (size 0.8) (drill 0.4) (layers "F.Cu" "B.Cu") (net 1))
 (via (at 134.62 83.185) (size 0.8) (drill 0.4) (layers "F.Cu" "B.Cu") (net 1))
 (segment (start 131.445 98.0225) (end 131.763275 97.704225) (width 0.25) (layer "B.Cu") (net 1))
 (segment (start 131.2125 74.93) (end 128.27 74.93) (width 0.25) (layer "B.Cu") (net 1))
 (segment (start 131.2125 90.17) (end 128.27 90.17) (width 0.25) (layer "B.Cu") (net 1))
 (segment (start 131.763275 97.704225) (end 133.899225 97.704225) (width 0.25) (layer "B.Cu") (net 1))
 (segment (start 131.445 90.4025) (end 131.2125 90.17) (width 0.25) (layer "B.Cu") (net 1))
 (segment (start 131.445 82.7825) (end 131.2125 82.55) (width 0.25) (layer "B.Cu") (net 1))
 (segment (start 133.899225 74.844225) (end 134.62 75.565) (width 0.25) (layer "B.Cu") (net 1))
 (segment (start 131.445 98.0225) (end 131.2125 97.79) (width 0.25) (layer "B.Cu") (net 1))
 (segment (start 131.445 75.1625) (end 131.763275 74.844225) (width 0.25) (layer "B.Cu") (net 1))
 (segment (start 131.445 82.7825) (end 131.763275 82.464225) (width 0.25) (layer "B.Cu") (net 1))
 (segment (start 131.763275 90.084225) (end 133.899225 90.084225) (width 0.25) (layer "B.Cu") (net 1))
 (segment (start 131.763275 82.464225) (end 133.899225 82.464225) (width 0.25) (layer "B.Cu") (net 1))
 (segment (start 131.2125 97.79) (end 128.27 97.79) (width 0.25) (layer "B.Cu") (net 1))
 (segment (start 133.899225 90.084225) (end 134.62 90.805) (width 0.25) (layer "B.Cu") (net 1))
 (segment (start 131.2125 82.55) (end 128.27 82.55) (width 0.25) (layer "B.Cu") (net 1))
 (segment (start 131.763275 74.844225) (end 133.899225 74.844225) (width 0.25) (layer "B.Cu") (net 1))
 (segment (start 133.899225 82.464225) (end 134.62 83.185) (width 0.25) (layer "B.Cu") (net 1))
 (segment (start 131.445 90.4025) (end 131.763275 90.084225) (width 0.25) (layer "B.Cu") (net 1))
 (segment (start 131.445 75.1625) (end 131.2125 74.93) (width 0.25) (layer "B.Cu") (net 1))
 (segment (start 133.899225 97.704225) (end 134.62 98.425) (width 0.25) (layer "B.Cu") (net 1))
 (segment (start 137.07 74.55) (end 137.07 74.991179) (width 0.25) (layer "F.Cu") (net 5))
 (segment (start 134.62 76.781847) (end 134.62 81.915) (width 0.25) (layer "F.Cu") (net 5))
 (segment (start 138.05 74.55) (end 140.97 77.47) (width 0.25) (layer "F.Cu") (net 5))
 (segment (start 137.07 74.991179) (end 136.495642 75.565537) (width 0.25) (layer "F.Cu") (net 5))
 (segment (start 137.07 74.55) (end 138.05 74.55) (width 0.25) (layer "F.Cu") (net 5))
 (via (at 136.495642 75.565537) (size 0.8) (drill 0.4) (layers "F.Cu" "B.Cu") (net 5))
 (via (at 134.62 81.915) (size 0.8) (drill 0.4) (layers "F.Cu" "B.Cu") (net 5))
 (via (at 134.62 76.781847) (size 0.8) (drill 0.4) (layers "F.Cu" "B.Cu") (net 5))
 (segment (start 134.62 76.781847) (end 135.279332 76.781847) (width 0.25) (layer "B.Cu") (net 5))
 (segment (start 135.279332 76.781847) (end 136.495642 75.565537) (width 0.25) (layer "B.Cu") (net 5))
 (segment (start 137.795 82.82) (end 138.065 82.55) (width 0.25) (layer "B.Cu") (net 5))
 (segment (start 138.065 82.55) (end 140.97 82.55) (width 0.25) (layer "B.Cu") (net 5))
 (segment (start 134.71 82.005) (end 136.98 82.005) (width 0.25) (layer "B.Cu") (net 5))
 (segment (start 134.62 81.915) (end 134.71 82.005) (width 0.25) (layer "B.Cu") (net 5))
 (segment (start 136.98 82.005) (end 137.795 82.82) (width 0.25) (layer "B.Cu") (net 5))
 (segment (start 132.17 77.85) (end 132.17 77.427451) (width 0.25) (layer "F.Cu") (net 6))
 (segment (start 132.17 77.427451) (end 132.766676 76.830775) (width 0.25) (layer "F.Cu") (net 6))
 (via (at 132.766676 76.830775) (size 0.8) (drill 0.4) (layers "F.Cu" "B.Cu") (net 6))
 (segment (start 137.488653 77.506347) (end 133.442248 77.506347) (width 0.25) (layer "B.Cu") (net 6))
 (segment (start 137.795 77.2) (end 137.488653 77.506347) (width 0.25) (layer "B.Cu") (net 6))
 (segment (start 133.442248 77.506347) (end 132.766676 76.830775) (width 0.25) (layer "B.Cu") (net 6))
 (segment (start 137.795 75.2) (end 138.065 74.93) (width 0.25) (layer "B.Cu") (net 11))
 (segment (start 138.065 74.93) (end 140.97 74.93) (width 0.25) (layer "B.Cu") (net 11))
 (segment (start 134.62 84.401847) (end 134.62 89.535) (width 0.25) (layer "F.Cu") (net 9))
 (segment (start 137.07 82.17) (end 138.05 82.17) (width 0.25) (layer "F.Cu") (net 9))
 (segment (start 138.05 82.17) (end 140.97 85.09) (width 0.25) (layer "F.Cu") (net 9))
 (segment (start 137.07 82.611179) (end 136.495642 83.185537) (width 0.25) (layer "F.Cu") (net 9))
 (segment (start 137.07 82.17) (end 137.07 82.611179) (width 0.25) (layer "F.Cu") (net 9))
 (via (at 136.495642 83.185537) (size 0.8) (drill 0.4) (layers "F.Cu" "B.Cu") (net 9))
 (via (at 134.62 84.401847) (size 0.8) (drill 0.4) (layers "F.Cu" "B.Cu") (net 9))
 (via (at 134.62 89.535) (size 0.8) (drill 0.4) (layers "F.Cu" "B.Cu") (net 9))
 (segment (start 134.62 89.535) (end 134.71 89.625) (width 0.25) (layer "B.Cu") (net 9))
 (segment (start 137.795 90.44) (end 138.065 90.17) (width 0.25) (layer "B.Cu") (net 9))
 (segment (start 136.98 89.625) (end 137.795 90.44) (width 0.25) (layer "B.Cu") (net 9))
 (segment (start 135.279332 84.401847) (end 136.495642 83.185537) (width 0.25) (layer "B.Cu") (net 9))
 (segment (start 134.62 84.401847) (end 135.279332 84.401847) (width 0.25) (layer "B.Cu") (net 9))
 (segment (start 138.065 90.17) (end 140.97 90.17) (width 0.25) (layer "B.Cu") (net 9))
 (segment (start 134.71 89.625) (end 136.98 89.625) (width 0.25) (layer "B.Cu") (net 9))
 (segment (start 132.17 85.047451) (end 132.766676 84.450775) (width 0.25) (layer "F.Cu") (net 10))
 (segment (start 132.17 85.47) (end 132.17 85.047451) (width 0.25) (layer "F.Cu") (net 10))
 (via (at 132.766676 84.450775) (size 0.8) (drill 0.4) (layers "F.Cu" "B.Cu") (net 10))
 (segment (start 137.488653 85.126347) (end 133.442248 85.126347) (width 0.25) (layer "B.Cu") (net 10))
 (segment (start 137.795 84.82) (end 137.488653 85.126347) (width 0.25) (layer "B.Cu") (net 10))
 (segment (start 133.442248 85.126347) (end 132.766676 84.450775) (width 0.25) (layer "B.Cu") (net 10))
 (segment (start 134.62 92.021847) (end 134.62 97.155) (width 0.25) (layer "F.Cu") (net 7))
 (segment (start 138.05 89.79) (end 140.97 92.71) (width 0.25) (layer "F.Cu") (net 7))
 (segment (start 137.07 89.79) (end 138.05 89.79) (width 0.25) (layer "F.Cu") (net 7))
 (segment (start 137.07 90.231179) (end 136.495642 90.805537) (width 0.25) (layer "F.Cu") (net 7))
 (segment (start 137.07 89.79) (end 137.07 90.231179) (width 0.25) (layer "F.Cu") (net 7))
 (via (at 134.62 92.021847) (size 0.8) (drill 0.4) (layers "F.Cu" "B.Cu") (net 7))
 (via (at 134.62 97.155) (size 0.8) (drill 0.4) (layers "F.Cu" "B.Cu") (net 7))
 (via (at 136.495642 90.805537) (size 0.8) (drill 0.4) (layers "F.Cu" "B.Cu") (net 7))
 (segment (start 134.62 92.021847) (end 135.279332 92.021847) (width 0.25) (layer "B.Cu") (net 7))
 (segment (start 134.62 97.155) (end 134.71 97.245) (width 0.25) (layer "B.Cu") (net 7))
 (segment (start 138.065 97.79) (end 140.97 97.79) (width 0.25) (layer "B.Cu") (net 7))
 (segment (start 135.279332 92.021847) (end 136.495642 90.805537) (width 0.25) (layer "B.Cu") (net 7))
 (segment (start 137.795 98.06) (end 138.065 97.79) (width 0.25) (layer "B.Cu") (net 7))
 (segment (start 134.71 97.245) (end 136.98 97.245) (width 0.25) (layer "B.Cu") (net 7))
 (segment (start 136.98 97.245) (end 137.795 98.06) (width 0.25) (layer "B.Cu") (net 7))
 (segment (start 132.17 92.667451) (end 132.766676 92.070775) (width 0.25) (layer "F.Cu") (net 8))
 (segment (start 132.17 93.09) (end 132.17 92.667451) (width 0.25) (layer "F.Cu") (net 8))
 (via (at 132.766676 92.070775) (size 0.8) (drill 0.4) (layers "F.Cu" "B.Cu") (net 8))
 (segment (start 137.795 92.44) (end 137.488653 92.746347) (width 0.25) (layer "B.Cu") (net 8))
 (segment (start 133.442248 92.746347) (end 132.766676 92.070775) (width 0.25) (layer "B.Cu") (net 8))
 (segment (start 137.488653 92.746347) (end 133.442248 92.746347) (width 0.25) (layer "B.Cu") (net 8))
 (segment (start 137.07 97.41) (end 138.05 97.41) (width 0.25) (layer "F.Cu") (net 2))
 (segment (start 138.05 97.41) (end 140.97 100.33) (width 0.25) (layer "F.Cu") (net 2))
 (segment (start 132.17 100.71) (end 132.17 100.287451) (width 0.25) (layer "F.Cu") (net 4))
 (segment (start 132.17 100.287451) (end 132.766676 99.690775) (width 0.25) (layer "F.Cu") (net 4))
 (via (at 132.766676 99.690775) (size 0.8) (drill 0.4) (layers "F.Cu" "B.Cu") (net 4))
 (segment (start 133.442248 100.366347) (end 132.766676 99.690775) (width 0.25) (layer "B.Cu") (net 4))
 (segment (start 137.795 100.06) (end 137.488653 100.366347) (width 0.25) (layer "B.Cu") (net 4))
 (segment (start 137.488653 100.366347) (end 133.442248 100.366347) (width 0.25) (layer "B.Cu") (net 4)))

